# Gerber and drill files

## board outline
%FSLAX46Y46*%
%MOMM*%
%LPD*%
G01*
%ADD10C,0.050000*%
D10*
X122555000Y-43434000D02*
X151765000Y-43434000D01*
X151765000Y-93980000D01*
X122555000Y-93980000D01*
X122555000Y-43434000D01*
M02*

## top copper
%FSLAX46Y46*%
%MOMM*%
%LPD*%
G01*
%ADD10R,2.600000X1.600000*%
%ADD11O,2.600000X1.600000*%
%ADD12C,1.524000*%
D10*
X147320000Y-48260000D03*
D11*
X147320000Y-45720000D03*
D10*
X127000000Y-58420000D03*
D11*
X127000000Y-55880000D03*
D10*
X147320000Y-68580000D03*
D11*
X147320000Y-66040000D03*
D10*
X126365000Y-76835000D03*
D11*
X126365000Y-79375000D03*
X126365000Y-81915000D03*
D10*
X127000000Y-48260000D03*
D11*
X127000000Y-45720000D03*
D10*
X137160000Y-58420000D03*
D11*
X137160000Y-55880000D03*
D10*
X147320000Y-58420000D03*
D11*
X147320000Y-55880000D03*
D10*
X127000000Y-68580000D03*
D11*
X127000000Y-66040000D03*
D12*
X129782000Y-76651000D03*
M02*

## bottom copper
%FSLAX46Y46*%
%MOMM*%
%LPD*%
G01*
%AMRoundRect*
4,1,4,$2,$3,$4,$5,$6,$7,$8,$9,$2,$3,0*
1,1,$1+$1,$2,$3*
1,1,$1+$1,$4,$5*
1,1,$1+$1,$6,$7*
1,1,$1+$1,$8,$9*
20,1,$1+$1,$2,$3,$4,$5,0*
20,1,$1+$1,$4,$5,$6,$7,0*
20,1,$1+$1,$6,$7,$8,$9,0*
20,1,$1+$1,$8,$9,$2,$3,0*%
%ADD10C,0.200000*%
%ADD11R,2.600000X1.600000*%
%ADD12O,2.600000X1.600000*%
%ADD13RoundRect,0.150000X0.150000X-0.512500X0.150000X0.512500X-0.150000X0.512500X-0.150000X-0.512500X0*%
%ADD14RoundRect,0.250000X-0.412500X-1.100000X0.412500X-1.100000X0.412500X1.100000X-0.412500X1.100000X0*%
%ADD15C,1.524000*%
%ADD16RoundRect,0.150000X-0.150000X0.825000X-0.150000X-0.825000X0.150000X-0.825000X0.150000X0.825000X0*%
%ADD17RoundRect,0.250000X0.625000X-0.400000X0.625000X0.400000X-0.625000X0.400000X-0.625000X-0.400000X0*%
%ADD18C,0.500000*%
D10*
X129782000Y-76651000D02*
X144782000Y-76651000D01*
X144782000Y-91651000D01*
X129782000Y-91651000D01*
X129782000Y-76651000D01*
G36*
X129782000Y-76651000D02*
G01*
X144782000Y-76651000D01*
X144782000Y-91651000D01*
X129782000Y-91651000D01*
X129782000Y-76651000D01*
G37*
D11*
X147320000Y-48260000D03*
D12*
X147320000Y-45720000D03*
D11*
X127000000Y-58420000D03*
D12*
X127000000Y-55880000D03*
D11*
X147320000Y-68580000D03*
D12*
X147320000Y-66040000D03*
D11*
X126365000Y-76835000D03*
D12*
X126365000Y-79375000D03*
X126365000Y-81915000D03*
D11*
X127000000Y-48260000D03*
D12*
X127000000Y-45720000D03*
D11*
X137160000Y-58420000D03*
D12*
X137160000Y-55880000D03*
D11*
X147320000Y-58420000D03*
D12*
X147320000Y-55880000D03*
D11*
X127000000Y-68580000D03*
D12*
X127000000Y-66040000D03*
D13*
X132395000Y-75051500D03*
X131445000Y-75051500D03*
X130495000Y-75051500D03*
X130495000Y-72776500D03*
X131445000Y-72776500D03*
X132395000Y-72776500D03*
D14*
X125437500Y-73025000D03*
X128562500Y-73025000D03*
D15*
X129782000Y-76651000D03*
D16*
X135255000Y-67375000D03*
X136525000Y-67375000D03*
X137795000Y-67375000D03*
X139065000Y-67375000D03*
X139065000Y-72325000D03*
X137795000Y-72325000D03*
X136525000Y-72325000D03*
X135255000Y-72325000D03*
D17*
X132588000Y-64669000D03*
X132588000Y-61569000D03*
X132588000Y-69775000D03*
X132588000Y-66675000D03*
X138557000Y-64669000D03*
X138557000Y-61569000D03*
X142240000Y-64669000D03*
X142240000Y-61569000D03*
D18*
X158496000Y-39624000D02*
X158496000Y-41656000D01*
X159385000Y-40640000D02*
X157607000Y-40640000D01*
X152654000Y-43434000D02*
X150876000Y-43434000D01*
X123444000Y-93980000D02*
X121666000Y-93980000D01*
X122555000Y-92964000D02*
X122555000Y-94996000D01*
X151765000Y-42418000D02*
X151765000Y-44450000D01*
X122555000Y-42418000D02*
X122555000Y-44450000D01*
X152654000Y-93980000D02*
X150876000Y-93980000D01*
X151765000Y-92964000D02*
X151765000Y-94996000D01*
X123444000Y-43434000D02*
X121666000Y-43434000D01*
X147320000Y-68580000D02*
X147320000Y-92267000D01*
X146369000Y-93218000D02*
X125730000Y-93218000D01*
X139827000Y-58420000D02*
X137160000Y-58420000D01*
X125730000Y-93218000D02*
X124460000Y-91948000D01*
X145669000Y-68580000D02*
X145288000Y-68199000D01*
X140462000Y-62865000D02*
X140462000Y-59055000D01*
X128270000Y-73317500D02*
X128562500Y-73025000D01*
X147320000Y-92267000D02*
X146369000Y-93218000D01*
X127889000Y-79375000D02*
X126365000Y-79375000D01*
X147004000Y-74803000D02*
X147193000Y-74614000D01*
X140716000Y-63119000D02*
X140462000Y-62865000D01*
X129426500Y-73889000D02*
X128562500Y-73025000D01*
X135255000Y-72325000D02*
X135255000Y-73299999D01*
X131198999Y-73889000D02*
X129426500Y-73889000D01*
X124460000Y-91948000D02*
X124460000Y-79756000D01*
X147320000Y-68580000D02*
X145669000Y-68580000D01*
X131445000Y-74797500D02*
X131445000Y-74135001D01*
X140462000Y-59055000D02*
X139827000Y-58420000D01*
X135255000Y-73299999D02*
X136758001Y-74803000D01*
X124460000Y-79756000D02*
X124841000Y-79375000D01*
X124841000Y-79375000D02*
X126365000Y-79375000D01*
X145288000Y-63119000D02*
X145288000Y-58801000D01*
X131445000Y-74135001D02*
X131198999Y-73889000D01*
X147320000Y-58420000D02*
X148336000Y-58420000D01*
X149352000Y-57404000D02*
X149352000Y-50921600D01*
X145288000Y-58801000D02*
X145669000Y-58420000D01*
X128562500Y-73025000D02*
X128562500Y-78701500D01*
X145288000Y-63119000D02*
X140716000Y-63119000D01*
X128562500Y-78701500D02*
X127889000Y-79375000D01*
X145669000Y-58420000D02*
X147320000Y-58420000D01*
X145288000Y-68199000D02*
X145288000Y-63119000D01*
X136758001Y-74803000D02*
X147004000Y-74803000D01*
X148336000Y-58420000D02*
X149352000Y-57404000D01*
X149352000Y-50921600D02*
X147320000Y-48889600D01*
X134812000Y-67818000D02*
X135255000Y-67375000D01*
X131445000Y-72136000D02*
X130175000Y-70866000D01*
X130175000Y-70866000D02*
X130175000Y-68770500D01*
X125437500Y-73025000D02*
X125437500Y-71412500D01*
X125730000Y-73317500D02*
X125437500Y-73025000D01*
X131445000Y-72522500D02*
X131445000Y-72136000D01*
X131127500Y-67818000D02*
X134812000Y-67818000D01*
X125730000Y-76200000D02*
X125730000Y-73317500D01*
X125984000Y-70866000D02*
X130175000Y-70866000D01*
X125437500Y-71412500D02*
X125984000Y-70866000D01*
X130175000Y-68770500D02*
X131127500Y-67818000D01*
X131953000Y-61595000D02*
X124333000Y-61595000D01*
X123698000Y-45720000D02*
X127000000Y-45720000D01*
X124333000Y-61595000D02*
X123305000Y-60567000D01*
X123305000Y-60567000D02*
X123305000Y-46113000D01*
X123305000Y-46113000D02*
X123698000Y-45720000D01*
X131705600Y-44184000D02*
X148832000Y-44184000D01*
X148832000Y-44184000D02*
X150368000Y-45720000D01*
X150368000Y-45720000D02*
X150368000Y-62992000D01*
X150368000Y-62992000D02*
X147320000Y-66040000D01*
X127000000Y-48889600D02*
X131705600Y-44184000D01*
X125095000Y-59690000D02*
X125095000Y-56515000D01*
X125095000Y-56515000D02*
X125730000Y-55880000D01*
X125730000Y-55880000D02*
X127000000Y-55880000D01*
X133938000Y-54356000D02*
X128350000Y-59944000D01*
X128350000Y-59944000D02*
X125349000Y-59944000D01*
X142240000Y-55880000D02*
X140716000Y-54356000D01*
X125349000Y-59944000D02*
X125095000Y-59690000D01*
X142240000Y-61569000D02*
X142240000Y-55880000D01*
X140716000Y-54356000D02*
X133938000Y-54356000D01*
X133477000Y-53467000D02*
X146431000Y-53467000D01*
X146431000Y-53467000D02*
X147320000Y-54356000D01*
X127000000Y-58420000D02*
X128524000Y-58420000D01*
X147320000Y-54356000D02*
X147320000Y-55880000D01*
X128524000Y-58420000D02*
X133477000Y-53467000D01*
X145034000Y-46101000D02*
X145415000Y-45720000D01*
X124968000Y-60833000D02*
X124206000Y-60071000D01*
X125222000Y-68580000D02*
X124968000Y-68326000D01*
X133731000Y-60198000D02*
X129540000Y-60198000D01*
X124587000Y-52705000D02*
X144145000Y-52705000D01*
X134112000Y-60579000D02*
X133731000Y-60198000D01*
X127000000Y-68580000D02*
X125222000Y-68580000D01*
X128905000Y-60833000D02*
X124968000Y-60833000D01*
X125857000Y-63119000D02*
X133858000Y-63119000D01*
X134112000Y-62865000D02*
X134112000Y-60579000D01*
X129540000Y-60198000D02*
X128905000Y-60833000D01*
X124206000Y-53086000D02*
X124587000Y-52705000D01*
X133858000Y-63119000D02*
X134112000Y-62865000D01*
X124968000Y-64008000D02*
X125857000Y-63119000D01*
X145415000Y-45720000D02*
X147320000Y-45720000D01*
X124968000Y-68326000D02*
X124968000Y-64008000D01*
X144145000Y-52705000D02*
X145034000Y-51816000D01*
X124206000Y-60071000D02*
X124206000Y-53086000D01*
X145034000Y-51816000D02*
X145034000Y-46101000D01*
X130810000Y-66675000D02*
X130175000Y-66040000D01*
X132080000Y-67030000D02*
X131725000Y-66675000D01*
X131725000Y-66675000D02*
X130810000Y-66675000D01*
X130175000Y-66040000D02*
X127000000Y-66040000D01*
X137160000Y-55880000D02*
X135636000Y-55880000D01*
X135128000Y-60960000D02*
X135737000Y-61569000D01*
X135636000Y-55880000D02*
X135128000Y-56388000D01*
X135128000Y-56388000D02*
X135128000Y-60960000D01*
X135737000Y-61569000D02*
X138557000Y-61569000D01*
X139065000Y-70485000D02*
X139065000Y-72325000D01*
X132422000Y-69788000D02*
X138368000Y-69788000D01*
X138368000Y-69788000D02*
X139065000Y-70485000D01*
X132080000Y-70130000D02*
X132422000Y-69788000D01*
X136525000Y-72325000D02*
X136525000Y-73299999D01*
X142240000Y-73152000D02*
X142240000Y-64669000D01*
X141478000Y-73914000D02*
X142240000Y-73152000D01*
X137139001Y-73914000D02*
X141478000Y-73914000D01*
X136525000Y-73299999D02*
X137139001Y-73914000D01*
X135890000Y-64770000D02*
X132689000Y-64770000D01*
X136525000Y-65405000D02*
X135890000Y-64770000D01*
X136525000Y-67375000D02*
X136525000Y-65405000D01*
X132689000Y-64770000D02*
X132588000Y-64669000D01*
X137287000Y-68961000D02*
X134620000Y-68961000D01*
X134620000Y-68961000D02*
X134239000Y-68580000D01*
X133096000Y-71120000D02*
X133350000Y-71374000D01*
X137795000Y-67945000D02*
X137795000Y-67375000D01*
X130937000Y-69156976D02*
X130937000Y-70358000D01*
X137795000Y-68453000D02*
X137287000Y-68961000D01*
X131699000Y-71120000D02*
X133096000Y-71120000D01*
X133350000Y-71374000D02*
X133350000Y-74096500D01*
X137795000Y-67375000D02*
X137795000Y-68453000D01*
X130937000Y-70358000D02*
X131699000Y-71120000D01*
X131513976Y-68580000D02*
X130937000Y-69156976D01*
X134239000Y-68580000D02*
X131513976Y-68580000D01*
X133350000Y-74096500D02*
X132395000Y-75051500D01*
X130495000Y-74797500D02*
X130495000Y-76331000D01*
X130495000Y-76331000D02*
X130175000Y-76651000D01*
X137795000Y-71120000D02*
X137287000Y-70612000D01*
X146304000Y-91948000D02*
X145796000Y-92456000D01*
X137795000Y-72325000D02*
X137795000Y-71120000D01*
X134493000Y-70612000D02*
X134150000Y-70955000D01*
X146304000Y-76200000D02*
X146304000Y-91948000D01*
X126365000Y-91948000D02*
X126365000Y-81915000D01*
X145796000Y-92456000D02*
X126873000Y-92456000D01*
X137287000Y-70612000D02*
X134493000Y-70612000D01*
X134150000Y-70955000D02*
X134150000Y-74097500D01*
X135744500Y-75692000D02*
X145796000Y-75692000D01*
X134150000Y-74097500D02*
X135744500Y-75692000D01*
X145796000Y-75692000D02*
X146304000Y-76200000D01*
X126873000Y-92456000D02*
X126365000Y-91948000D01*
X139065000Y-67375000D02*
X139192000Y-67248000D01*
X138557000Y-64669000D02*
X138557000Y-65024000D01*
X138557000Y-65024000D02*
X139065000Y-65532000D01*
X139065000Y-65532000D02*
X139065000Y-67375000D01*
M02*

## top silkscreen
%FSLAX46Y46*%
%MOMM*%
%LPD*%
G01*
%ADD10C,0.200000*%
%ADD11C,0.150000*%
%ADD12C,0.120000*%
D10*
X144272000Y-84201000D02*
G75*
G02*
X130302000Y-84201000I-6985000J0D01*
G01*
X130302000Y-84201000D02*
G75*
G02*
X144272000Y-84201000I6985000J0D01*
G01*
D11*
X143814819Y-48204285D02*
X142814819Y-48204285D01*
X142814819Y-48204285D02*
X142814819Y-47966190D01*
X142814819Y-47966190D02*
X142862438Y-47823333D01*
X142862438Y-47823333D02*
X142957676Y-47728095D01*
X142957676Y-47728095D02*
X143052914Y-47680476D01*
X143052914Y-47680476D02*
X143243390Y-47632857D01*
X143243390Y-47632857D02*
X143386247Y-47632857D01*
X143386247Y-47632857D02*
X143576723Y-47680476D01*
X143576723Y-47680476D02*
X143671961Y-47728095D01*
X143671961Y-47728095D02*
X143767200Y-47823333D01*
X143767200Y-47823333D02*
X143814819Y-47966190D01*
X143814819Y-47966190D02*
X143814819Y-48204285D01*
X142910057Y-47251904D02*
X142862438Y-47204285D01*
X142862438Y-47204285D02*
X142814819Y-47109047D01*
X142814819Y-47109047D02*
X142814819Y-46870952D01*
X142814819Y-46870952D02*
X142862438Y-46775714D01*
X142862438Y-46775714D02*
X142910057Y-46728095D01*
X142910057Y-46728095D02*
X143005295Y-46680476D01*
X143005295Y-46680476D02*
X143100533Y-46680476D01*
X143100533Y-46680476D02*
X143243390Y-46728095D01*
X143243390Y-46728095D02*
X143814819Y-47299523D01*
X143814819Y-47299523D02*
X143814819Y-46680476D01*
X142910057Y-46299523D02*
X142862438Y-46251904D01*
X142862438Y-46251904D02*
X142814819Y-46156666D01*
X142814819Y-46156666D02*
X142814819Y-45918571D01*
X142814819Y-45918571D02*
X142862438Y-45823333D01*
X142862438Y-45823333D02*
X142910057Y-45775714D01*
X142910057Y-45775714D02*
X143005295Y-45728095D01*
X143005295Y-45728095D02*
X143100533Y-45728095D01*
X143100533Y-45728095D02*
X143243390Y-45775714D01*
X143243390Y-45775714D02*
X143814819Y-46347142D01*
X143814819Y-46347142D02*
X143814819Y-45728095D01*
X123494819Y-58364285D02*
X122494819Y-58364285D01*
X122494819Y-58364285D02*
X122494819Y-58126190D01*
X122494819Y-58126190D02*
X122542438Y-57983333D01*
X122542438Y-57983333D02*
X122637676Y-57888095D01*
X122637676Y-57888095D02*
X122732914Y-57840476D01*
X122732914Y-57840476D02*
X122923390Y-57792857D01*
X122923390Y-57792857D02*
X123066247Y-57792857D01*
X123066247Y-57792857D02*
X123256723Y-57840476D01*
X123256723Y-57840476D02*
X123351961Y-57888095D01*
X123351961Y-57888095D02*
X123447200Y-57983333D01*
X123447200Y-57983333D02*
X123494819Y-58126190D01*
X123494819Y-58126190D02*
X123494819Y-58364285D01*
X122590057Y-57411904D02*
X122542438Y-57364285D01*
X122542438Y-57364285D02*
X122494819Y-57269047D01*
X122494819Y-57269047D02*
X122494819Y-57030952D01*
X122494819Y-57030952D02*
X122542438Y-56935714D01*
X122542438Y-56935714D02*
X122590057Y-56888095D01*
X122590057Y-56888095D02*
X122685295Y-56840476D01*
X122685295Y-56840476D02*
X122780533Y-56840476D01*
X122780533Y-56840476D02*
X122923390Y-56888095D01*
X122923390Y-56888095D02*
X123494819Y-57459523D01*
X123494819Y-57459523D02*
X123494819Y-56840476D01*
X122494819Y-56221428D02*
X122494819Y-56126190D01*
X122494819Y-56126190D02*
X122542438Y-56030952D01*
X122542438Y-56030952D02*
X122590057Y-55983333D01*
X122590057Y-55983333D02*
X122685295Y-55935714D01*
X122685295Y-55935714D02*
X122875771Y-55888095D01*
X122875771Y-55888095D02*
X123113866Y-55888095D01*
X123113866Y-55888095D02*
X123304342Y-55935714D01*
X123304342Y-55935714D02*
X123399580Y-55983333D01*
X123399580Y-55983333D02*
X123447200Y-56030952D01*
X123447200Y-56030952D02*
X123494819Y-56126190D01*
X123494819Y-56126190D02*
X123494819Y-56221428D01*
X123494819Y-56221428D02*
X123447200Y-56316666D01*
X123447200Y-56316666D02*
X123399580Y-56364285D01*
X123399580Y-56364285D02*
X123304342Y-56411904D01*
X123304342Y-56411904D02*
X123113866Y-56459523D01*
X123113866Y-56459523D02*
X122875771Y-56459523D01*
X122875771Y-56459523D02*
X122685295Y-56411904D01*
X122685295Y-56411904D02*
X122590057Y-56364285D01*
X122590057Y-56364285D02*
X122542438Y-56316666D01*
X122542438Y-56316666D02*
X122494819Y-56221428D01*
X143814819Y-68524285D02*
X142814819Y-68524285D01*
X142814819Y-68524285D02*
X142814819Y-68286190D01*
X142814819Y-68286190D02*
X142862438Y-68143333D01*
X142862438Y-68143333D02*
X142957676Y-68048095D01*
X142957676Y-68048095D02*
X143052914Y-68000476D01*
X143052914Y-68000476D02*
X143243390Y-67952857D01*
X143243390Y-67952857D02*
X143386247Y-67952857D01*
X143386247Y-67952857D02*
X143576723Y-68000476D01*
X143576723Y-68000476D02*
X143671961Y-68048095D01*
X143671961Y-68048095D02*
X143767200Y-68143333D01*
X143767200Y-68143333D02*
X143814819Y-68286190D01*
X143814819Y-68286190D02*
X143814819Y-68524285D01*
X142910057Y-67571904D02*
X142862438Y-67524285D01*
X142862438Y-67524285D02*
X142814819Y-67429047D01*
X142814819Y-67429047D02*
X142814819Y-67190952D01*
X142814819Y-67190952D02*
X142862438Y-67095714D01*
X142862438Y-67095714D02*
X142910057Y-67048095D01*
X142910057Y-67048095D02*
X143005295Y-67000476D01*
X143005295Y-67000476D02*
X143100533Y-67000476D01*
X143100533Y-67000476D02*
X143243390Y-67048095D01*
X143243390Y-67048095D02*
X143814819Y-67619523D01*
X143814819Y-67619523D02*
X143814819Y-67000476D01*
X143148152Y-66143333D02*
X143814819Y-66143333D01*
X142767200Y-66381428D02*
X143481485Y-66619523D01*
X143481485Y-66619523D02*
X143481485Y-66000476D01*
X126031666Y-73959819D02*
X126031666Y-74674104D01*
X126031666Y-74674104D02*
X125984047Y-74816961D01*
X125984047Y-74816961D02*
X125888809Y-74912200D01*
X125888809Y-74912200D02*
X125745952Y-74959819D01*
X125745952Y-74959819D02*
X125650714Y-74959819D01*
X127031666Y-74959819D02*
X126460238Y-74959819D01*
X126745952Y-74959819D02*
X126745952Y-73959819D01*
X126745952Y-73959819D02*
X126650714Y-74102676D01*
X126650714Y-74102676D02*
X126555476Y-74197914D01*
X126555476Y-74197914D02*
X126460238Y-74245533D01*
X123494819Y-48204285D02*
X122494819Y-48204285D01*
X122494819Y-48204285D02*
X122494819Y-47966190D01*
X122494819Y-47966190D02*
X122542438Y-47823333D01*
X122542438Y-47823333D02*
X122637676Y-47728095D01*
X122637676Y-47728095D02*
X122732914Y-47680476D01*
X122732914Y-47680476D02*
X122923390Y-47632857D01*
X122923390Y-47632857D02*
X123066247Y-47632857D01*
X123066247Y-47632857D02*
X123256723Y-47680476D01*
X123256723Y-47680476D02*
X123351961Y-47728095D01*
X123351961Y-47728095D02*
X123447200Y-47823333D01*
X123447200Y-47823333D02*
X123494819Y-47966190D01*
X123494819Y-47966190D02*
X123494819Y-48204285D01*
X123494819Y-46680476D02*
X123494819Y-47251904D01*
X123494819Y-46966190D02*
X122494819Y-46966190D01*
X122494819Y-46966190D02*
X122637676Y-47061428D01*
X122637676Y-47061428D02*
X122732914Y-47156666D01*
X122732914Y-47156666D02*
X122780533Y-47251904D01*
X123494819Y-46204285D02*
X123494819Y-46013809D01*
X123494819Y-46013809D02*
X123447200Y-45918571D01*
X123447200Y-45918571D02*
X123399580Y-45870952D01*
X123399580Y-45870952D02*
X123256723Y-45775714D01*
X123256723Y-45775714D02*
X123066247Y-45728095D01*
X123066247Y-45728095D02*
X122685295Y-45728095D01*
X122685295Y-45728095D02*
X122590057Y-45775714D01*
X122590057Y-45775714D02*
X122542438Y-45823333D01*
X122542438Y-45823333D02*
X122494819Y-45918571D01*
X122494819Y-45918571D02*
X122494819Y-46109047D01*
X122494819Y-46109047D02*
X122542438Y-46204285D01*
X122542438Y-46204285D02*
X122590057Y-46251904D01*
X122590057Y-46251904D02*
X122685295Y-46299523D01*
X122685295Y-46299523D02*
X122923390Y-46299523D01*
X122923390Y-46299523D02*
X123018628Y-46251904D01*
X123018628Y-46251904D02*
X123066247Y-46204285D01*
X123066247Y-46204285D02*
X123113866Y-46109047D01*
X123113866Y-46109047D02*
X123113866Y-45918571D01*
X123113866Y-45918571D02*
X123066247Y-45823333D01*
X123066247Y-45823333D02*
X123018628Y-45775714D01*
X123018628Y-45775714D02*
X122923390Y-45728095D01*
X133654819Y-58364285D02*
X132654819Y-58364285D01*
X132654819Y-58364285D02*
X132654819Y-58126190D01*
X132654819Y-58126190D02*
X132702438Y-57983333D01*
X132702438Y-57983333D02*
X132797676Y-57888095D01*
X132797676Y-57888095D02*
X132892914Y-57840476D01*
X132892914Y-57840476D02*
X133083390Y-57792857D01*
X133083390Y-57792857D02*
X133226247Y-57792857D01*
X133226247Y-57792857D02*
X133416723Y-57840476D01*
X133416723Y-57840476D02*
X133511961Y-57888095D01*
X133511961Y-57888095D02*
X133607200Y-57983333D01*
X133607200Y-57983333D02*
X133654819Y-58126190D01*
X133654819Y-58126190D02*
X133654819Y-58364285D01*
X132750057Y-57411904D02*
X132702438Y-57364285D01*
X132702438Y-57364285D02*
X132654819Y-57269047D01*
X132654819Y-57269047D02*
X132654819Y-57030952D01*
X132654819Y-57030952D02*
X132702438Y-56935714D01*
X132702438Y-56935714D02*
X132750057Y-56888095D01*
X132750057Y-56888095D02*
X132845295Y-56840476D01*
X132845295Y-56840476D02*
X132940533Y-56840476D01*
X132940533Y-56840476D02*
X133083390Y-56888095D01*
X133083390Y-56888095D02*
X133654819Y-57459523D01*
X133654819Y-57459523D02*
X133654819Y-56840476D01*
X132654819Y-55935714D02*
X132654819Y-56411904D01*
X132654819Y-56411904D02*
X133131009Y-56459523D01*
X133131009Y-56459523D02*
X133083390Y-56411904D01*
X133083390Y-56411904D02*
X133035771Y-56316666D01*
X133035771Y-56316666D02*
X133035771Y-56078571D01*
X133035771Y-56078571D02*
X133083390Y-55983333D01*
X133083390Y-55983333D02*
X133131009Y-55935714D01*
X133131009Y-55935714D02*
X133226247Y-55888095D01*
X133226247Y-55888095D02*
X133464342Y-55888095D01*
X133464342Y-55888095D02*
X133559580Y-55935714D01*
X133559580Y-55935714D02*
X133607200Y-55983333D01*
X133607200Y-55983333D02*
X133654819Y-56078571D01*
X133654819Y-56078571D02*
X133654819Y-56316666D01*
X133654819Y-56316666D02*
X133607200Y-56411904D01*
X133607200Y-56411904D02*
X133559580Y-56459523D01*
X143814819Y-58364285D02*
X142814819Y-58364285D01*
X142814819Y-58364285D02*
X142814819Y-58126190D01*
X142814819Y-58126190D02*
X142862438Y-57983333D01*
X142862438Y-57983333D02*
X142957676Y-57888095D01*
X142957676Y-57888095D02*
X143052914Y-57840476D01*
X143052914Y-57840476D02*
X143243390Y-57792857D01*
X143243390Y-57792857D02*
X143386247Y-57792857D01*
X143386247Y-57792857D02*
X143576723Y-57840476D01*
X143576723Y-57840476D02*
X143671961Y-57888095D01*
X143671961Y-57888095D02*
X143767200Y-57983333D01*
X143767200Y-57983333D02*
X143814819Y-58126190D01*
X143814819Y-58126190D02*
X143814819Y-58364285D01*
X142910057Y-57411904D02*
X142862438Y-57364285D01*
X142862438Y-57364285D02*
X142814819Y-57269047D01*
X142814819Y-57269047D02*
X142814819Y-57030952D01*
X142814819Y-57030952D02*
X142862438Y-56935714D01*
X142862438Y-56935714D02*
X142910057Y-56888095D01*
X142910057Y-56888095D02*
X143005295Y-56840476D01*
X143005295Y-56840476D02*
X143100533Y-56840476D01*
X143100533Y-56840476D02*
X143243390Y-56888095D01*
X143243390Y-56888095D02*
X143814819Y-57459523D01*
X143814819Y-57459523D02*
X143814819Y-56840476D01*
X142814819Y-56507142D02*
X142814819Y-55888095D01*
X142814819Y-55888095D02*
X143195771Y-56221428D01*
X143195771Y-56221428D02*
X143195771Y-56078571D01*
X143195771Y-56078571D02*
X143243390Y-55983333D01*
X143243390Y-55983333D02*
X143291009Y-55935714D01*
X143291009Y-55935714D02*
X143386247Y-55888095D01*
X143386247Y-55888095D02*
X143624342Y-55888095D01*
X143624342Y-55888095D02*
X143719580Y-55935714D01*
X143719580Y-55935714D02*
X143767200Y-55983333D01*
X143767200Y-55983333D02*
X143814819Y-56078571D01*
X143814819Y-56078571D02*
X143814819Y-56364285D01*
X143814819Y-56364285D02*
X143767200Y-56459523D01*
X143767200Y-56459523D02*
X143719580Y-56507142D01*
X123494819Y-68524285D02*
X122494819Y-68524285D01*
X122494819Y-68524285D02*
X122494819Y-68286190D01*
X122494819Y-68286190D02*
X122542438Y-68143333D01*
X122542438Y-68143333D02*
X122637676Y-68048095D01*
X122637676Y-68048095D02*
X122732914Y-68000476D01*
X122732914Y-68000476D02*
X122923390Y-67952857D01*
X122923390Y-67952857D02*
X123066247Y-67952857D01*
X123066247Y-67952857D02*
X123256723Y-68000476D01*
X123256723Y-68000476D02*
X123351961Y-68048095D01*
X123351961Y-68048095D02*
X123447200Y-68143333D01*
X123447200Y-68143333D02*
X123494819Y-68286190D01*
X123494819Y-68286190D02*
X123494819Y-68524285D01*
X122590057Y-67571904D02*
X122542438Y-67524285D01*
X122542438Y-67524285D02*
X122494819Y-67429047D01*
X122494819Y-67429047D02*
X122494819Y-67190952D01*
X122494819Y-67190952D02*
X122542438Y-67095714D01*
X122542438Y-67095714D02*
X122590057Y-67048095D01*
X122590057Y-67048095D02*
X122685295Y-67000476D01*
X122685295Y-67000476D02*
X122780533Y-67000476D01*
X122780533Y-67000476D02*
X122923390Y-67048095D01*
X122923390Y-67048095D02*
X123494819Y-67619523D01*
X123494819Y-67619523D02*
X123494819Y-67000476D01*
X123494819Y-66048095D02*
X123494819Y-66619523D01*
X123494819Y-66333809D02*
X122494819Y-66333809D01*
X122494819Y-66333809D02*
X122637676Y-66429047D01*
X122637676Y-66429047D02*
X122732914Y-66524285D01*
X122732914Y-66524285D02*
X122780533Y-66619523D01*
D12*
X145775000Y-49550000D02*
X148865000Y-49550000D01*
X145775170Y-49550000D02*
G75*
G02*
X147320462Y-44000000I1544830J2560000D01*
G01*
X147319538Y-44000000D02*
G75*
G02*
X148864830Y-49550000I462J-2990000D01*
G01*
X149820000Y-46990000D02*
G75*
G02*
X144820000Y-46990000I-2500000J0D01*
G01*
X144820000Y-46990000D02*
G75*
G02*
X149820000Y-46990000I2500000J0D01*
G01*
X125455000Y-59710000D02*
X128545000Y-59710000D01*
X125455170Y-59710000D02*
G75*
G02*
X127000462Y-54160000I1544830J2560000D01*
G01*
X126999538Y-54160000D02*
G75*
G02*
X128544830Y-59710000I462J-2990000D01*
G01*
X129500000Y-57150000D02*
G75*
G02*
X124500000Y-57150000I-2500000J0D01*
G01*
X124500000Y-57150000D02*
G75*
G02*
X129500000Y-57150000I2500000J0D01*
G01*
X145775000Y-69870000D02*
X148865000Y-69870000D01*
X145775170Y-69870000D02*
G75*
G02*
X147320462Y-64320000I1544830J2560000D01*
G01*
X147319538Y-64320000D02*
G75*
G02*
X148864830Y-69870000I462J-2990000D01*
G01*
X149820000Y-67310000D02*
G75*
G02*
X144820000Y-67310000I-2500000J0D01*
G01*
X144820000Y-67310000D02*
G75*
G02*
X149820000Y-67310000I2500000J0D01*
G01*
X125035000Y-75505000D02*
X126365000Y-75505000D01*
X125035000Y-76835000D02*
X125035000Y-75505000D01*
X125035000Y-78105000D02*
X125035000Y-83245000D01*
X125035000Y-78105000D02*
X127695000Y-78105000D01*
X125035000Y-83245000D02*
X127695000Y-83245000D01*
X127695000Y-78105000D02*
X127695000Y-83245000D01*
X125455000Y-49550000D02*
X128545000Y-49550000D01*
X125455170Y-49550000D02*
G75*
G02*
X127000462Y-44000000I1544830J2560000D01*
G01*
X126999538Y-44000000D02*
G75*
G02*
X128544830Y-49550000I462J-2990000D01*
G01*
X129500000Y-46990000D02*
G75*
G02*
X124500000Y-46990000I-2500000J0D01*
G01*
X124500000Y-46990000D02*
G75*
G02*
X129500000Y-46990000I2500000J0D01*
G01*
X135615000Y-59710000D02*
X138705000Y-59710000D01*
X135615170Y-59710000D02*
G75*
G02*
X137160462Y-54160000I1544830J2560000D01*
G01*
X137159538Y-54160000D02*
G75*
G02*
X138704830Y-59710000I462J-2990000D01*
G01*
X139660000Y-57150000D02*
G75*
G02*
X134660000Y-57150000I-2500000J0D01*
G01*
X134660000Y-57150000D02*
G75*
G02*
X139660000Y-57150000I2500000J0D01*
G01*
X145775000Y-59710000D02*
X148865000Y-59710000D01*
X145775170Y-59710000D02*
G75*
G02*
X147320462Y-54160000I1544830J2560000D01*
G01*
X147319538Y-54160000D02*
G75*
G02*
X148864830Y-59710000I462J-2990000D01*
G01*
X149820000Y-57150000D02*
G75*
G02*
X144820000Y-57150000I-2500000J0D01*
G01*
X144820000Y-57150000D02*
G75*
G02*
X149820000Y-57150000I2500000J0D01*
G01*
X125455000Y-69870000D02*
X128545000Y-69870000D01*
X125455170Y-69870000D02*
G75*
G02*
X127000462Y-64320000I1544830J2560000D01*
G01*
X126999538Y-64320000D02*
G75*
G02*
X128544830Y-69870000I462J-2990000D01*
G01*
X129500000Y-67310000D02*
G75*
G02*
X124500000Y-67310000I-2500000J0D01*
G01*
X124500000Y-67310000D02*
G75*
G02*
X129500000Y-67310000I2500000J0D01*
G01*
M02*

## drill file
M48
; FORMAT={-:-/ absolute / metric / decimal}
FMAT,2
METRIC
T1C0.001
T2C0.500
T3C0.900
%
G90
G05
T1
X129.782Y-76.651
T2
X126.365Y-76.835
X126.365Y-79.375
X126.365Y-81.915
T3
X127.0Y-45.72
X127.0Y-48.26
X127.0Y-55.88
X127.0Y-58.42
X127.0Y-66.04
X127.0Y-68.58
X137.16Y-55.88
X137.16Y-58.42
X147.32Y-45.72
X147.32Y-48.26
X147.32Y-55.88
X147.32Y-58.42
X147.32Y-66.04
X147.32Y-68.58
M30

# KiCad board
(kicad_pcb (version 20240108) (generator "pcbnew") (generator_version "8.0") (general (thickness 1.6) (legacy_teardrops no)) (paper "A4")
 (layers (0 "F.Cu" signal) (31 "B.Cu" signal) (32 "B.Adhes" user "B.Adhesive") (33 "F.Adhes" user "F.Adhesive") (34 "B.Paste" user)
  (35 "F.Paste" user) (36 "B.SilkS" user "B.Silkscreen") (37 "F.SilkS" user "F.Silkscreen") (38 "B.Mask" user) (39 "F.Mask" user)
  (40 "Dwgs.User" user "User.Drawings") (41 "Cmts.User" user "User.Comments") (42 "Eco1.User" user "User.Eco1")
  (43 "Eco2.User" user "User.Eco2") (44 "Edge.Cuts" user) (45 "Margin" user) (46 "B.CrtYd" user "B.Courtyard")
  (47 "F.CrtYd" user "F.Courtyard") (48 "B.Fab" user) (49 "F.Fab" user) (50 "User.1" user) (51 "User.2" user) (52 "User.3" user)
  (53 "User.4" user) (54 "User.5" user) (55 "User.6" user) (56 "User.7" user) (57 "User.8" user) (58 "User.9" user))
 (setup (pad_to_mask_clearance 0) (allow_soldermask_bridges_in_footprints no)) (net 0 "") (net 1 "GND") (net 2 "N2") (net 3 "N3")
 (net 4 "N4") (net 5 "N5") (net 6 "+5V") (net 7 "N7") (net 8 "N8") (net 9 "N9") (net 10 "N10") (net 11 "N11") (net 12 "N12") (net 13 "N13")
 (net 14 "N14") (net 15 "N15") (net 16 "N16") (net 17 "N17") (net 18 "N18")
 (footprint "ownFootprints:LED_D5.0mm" (layer "F.Cu") (at 147.32 48.26 90)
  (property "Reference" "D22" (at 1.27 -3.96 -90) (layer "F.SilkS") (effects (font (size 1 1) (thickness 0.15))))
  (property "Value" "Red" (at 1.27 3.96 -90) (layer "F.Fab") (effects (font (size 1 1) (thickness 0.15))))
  (fp_line (start -1.29 -1.545) (end -1.29 1.545) (stroke (width 0.12) (type solid)) (layer "F.SilkS"))
  (fp_arc (start -1.29 -1.54483) (mid 2.072002 -2.880433) (end 4.26 0.000462) (stroke (width 0.12) (type solid)) (layer "F.SilkS"))
  (fp_arc (start 4.26 -0.000462) (mid 2.072002 2.880433) (end -1.29 1.54483) (stroke (width 0.12) (type solid)) (layer "F.SilkS"))
  (fp_circle (center 1.27 0) (end 3.77 0) (stroke (width 0.12) (type solid)) (fill none) (layer "F.SilkS"))
  (pad "1" thru_hole rect (at 0 0 90) (size 1.6 2.6) (drill 0.9) (layers "*.Cu" "*.Mask") (remove_unused_layers no) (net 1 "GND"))
  (pad "2" thru_hole oval (at 2.54 0 90) (size 1.6 2.6) (drill 0.9) (layers "*.Cu" "*.Mask") (remove_unused_layers no) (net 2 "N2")))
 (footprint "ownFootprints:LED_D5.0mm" (layer "F.Cu") (at 127 58.42 90)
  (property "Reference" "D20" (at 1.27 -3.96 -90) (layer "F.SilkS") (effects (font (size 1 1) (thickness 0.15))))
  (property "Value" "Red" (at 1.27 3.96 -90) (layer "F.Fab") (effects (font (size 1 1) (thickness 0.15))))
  (fp_line (start -1.29 -1.545) (end -1.29 1.545) (stroke (width 0.12) (type solid)) (layer "F.SilkS"))
  (fp_arc (start -1.29 -1.54483) (mid 2.072002 -2.880433) (end 4.26 0.000462) (stroke (width 0.12) (type solid)) (layer "F.SilkS"))
  (fp_arc (start 4.26 -0.000462) (mid 2.072002 2.880433) (end -1.29 1.54483) (stroke (width 0.12) (type solid)) (layer "F.SilkS"))
  (fp_circle (center 1.27 0) (end 3.77 0) (stroke (width 0.12) (type solid)) (fill none) (layer "F.SilkS"))
  (pad "1" thru_hole rect (at 0 0 90) (size 1.6 2.6) (drill 0.9) (layers "*.Cu" "*.Mask") (remove_unused_layers no) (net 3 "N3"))
  (pad "2" thru_hole oval (at 2.54 0 90) (size 1.6 2.6) (drill 0.9) (layers "*.Cu" "*.Mask") (remove_unused_layers no) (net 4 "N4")))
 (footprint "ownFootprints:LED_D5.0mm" (layer "F.Cu") (at 147.32 68.58 90)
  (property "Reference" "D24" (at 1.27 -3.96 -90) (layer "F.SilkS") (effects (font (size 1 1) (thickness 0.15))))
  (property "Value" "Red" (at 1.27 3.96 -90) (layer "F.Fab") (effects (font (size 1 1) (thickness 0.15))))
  (fp_line (start -1.29 -1.545) (end -1.29 1.545) (stroke (width 0.12) (type solid)) (layer "F.SilkS"))
  (fp_arc (start -1.29 -1.54483) (mid 2.072002 -2.880433) (end 4.26 0.000462) (stroke (width 0.12) (type solid)) (layer "F.SilkS"))
  (fp_arc (start 4.26 -0.000462) (mid 2.072002 2.880433) (end -1.29 1.54483) (stroke (width 0.12) (type solid)) (layer "F.SilkS"))
  (fp_circle (center 1.27 0) (end 3.77 0) (stroke (width 0.12) (type solid)) (fill none) (layer "F.SilkS"))
  (pad "1" thru_hole rect (at 0 0 90) (size 1.6 2.6) (drill 0.9) (layers "*.Cu" "*.Mask") (remove_unused_layers no) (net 1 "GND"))
  (pad "2" thru_hole oval (at 2.54 0 90) (size 1.6 2.6) (drill 0.9) (layers "*.Cu" "*.Mask") (remove_unused_layers no) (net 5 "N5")))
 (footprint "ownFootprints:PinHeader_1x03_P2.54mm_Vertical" (layer "F.Cu") (at 126.365 76.835)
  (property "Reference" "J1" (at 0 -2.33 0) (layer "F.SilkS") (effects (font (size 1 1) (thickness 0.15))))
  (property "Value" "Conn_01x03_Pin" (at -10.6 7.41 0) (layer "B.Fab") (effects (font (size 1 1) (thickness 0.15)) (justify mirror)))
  (fp_line (start -1.33 -1.33) (end 0 -1.33) (stroke (width 0.12) (type solid)) (layer "F.SilkS"))
  (fp_line (start -1.33 0) (end -1.33 -1.33) (stroke (width 0.12) (type solid)) (layer "F.SilkS"))
  (fp_line (start -1.33 1.27) (end -1.33 6.41) (stroke (width 0.12) (type solid)) (layer "F.SilkS"))
  (fp_line (start -1.33 1.27) (end 1.33 1.27) (stroke (width 0.12) (type solid)) (layer "F.SilkS"))
  (fp_line (start -1.33 6.41) (end 1.33 6.41) (stroke (width 0.12) (type solid)) (layer "F.SilkS"))
  (fp_line (start 1.33 1.27) (end 1.33 6.41) (stroke (width 0.12) (type solid)) (layer "F.SilkS"))
  (pad "1" thru_hole rect (at 0 0) (size 2.6 1.6) (drill 0.5) (layers "*.Cu" "*.Mask") (remove_unused_layers no) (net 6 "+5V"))
  (pad "2" thru_hole oval (at 0 2.54) (size 2.6 1.6) (drill 0.5) (layers "*.Cu" "*.Mask") (remove_unused_layers no) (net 1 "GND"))
  (pad "3" thru_hole oval (at 0 5.08) (size 2.6 1.6) (drill 0.5) (layers "*.Cu" "*.Mask") (remove_unused_layers no) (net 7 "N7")))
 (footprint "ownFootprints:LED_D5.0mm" (layer "F.Cu") (at 127 48.26 90)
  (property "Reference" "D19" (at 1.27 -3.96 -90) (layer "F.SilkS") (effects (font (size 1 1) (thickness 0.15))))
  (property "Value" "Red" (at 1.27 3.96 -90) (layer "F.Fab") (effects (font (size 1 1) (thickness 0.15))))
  (fp_line (start -1.29 -1.545) (end -1.29 1.545) (stroke (width 0.12) (type solid)) (layer "F.SilkS"))
  (fp_arc (start -1.29 -1.54483) (mid 2.072002 -2.880433) (end 4.26 0.000462) (stroke (width 0.12) (type solid)) (layer "F.SilkS"))
  (fp_arc (start 4.26 -0.000462) (mid 2.072002 2.880433) (end -1.29 1.54483) (stroke (width 0.12) (type solid)) (layer "F.SilkS"))
  (fp_circle (center 1.27 0) (end 3.77 0) (stroke (width 0.12) (type solid)) (fill none) (layer "F.SilkS"))
  (pad "1" thru_hole rect (at 0 0 90) (size 1.6 2.6) (drill 0.9) (layers "*.Cu" "*.Mask") (remove_unused_layers no) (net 5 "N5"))
  (pad "2" thru_hole oval (at 2.54 0 90) (size 1.6 2.6) (drill 0.9) (layers "*.Cu" "*.Mask") (remove_unused_layers no) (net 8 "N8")))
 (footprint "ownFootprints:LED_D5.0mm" (layer "F.Cu") (at 137.16 58.42 90)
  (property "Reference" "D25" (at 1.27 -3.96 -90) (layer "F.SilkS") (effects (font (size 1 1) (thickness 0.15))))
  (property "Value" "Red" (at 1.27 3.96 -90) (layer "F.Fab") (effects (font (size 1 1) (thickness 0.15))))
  (fp_line (start -1.29 -1.545) (end -1.29 1.545) (stroke (width 0.12) (type solid)) (layer "F.SilkS"))
  (fp_arc (start -1.29 -1.54483) (mid 2.072002 -2.880433) (end 4.26 0.000462) (stroke (width 0.12) (type solid)) (layer "F.SilkS"))
  (fp_arc (start 4.26 -0.000462) (mid 2.072002 2.880433) (end -1.29 1.54483) (stroke (width 0.12) (type solid)) (layer "F.SilkS"))
  (fp_circle (center 1.27 0) (end 3.77 0) (stroke (width 0.12) (type solid)) (fill none) (layer "F.SilkS"))
  (pad "1" thru_hole rect (at 0 0 90) (size 1.6 2.6) (drill 0.9) (layers "*.Cu" "*.Mask") (remove_unused_layers no) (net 1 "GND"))
  (pad "2" thru_hole oval (at 2.54 0 90) (size 1.6 2.6) (drill 0.9) (layers "*.Cu" "*.Mask") (remove_unused_layers no) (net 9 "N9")))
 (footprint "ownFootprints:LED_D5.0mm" (layer "F.Cu") (at 147.32 58.42 90)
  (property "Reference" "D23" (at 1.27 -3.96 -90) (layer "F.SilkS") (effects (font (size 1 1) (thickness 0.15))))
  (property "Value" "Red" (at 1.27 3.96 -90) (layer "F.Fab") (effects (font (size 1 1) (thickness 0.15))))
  (fp_line (start -1.29 -1.545) (end -1.29 1.545) (stroke (width 0.12) (type solid)) (layer "F.SilkS"))
  (fp_arc (start -1.29 -1.54483) (mid 2.072002 -2.880433) (end 4.26 0.000462) (stroke (width 0.12) (type solid)) (layer "F.SilkS"))
  (fp_arc (start 4.26 -0.000462) (mid 2.072002 2.880433) (end -1.29 1.54483) (stroke (width 0.12) (type solid)) (layer "F.SilkS"))
  (fp_circle (center 1.27 0) (end 3.77 0) (stroke (width 0.12) (type solid)) (fill none) (layer "F.SilkS"))
  (pad "1" thru_hole rect (at 0 0 90) (size 1.6 2.6) (drill 0.9) (layers "*.Cu" "*.Mask") (remove_unused_layers no) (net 1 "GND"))
  (pad "2" thru_hole oval (at 2.54 0 90) (size 1.6 2.6) (drill 0.9) (layers "*.Cu" "*.Mask") (remove_unused_layers no) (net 3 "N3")))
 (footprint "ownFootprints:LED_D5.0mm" (layer "F.Cu") (at 127 68.58 90)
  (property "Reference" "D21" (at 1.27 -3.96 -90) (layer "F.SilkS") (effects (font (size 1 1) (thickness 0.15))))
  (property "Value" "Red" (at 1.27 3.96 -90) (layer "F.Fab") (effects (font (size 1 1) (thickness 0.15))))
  (fp_line (start -1.29 -1.545) (end -1.29 1.545) (stroke (width 0.12) (type solid)) (layer "F.SilkS"))
  (fp_arc (start -1.29 -1.54483) (mid 2.072002 -2.880433) (end 4.26 0.000462) (stroke (width 0.12) (type solid)) (layer "F.SilkS"))
  (fp_arc (start 4.26 -0.000462) (mid 2.072002 2.880433) (end -1.29 1.54483) (stroke (width 0.12) (type solid)) (layer "F.SilkS"))
  (fp_circle (center 1.27 0) (end 3.77 0) (stroke (width 0.12) (type solid)) (fill none) (layer "F.SilkS"))
  (pad "1" thru_hole rect (at 0 0 90) (size 1.6 2.6) (drill 0.9) (layers "*.Cu" "*.Mask") (remove_unused_layers no) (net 2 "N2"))
  (pad "2" thru_hole oval (at 2.54 0 90) (size 1.6 2.6) (drill 0.9) (layers "*.Cu" "*.Mask") (remove_unused_layers no) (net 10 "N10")))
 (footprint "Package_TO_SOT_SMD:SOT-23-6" (layer "B.Cu") (at 131.445 73.914 90)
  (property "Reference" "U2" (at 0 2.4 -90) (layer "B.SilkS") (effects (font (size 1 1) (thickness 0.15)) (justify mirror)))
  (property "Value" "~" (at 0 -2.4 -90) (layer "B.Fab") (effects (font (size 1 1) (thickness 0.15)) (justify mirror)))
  (pad "1" smd roundrect (at -1.1375 0.95 90) (size 1.325 0.6) (layers "B.Cu" "B.Paste" "B.Mask") (roundrect_rratio 0.25) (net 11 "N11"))
  (pad "2" smd roundrect (at -1.1375 0 90) (size 1.325 0.6) (layers "B.Cu" "B.Paste" "B.Mask") (roundrect_rratio 0.25) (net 1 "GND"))
  (pad "3" smd roundrect (at -1.1375 -0.95 90) (size 1.325 0.6) (layers "B.Cu" "B.Paste" "B.Mask") (roundrect_rratio 0.25) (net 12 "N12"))
  (pad "4" smd roundrect (at 1.1375 -0.95 90) (size 1.325 0.6) (layers "B.Cu" "B.Paste" "B.Mask") (roundrect_rratio 0.25) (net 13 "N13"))
  (pad "5" smd roundrect (at 1.1375 0 90) (size 1.325 0.6) (layers "B.Cu" "B.Paste" "B.Mask") (roundrect_rratio 0.25) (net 6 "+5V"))
  (pad "6" smd roundrect (at 1.1375 0.95 90) (size 1.325 0.6) (layers "B.Cu" "B.Paste" "B.Mask") (roundrect_rratio 0.25) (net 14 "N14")))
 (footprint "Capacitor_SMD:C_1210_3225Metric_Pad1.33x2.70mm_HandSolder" (layer "B.Cu") (at 127 73.025)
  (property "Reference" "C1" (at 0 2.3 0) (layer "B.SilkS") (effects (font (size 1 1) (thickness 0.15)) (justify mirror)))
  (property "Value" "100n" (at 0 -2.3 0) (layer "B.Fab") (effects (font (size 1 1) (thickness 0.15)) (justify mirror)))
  (pad "1" smd roundrect (at -1.5625 0) (size 1.325 2.7) (layers "B.Cu" "B.Paste" "B.Mask") (roundrect_rratio 0.188679) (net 6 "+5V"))
  (pad "2" smd roundrect (at 1.5625 0) (size 1.325 2.7) (layers "B.Cu" "B.Paste" "B.Mask") (roundrect_rratio 0.188679) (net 1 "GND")))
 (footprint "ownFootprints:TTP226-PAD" (layer "B.Cu") (at 119.782 80.651 -90)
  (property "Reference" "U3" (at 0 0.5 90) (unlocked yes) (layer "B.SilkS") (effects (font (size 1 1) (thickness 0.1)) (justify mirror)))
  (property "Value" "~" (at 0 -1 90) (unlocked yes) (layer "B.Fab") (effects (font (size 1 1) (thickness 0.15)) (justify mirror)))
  (fp_rect (start 11 -25) (end -4 -10) (stroke (width 0.2) (type solid)) (fill solid) (layer "B.Cu"))
  (pad "1" thru_hole circle (at -4 -10 270) (size 1.524 1.524) (drill 0.001) (layers "*.Cu" "B.Mask") (remove_unused_layers no)
   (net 12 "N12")))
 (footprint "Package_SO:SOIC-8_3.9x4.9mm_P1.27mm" (layer "B.Cu") (at 137.16 69.85 -90)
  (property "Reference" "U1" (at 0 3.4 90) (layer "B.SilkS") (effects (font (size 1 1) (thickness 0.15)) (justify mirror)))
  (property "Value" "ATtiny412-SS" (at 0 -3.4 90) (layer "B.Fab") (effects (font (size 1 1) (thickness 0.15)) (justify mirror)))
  (pad "1" smd roundrect (at -2.475 1.905 270) (size 1.95 0.6) (layers "B.Cu" "B.Paste" "B.Mask") (roundrect_rratio 0.25) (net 6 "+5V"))
  (pad "2" smd roundrect (at -2.475 0.635 270) (size 1.95 0.6) (layers "B.Cu" "B.Paste" "B.Mask") (roundrect_rratio 0.25) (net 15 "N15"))
  (pad "3" smd roundrect (at -2.475 -0.635 270) (size 1.95 0.6) (layers "B.Cu" "B.Paste" "B.Mask") (roundrect_rratio 0.25) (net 11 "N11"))
  (pad "4" smd roundrect (at -2.475 -1.905 270) (size 1.95 0.6) (layers "B.Cu" "B.Paste" "B.Mask") (roundrect_rratio 0.25) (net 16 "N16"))
  (pad "5" smd roundrect (at 2.475 -1.905 270) (size 1.95 0.6) (layers "B.Cu" "B.Paste" "B.Mask") (roundrect_rratio 0.25) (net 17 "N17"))
  (pad "6" smd roundrect (at 2.475 -0.635 270) (size 1.95 0.6) (layers "B.Cu" "B.Paste" "B.Mask") (roundrect_rratio 0.25) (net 7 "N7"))
  (pad "7" smd roundrect (at 2.475 0.635 270) (size 1.95 0.6) (layers "B.Cu" "B.Paste" "B.Mask") (roundrect_rratio 0.25) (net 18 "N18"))
  (pad "8" smd roundrect (at 2.475 1.905 270) (size 1.95 0.6) (layers "B.Cu" "B.Paste" "B.Mask") (roundrect_rratio 0.25) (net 1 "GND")))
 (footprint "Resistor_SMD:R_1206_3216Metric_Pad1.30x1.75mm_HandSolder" (layer "B.Cu") (at 132.588 63.119 90)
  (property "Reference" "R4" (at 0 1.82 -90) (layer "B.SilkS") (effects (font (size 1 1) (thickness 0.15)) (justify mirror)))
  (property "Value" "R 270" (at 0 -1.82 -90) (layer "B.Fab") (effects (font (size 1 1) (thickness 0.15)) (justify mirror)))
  (pad "1" smd roundrect (at -1.55 0 90) (size 1.3 1.75) (layers "B.Cu" "B.Paste" "B.Mask") (roundrect_rratio 0.192308) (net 15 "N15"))
  (pad "2" smd roundrect (at 1.55 0 90) (size 1.3 1.75) (layers "B.Cu" "B.Paste" "B.Mask") (roundrect_rratio 0.192308) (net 8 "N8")))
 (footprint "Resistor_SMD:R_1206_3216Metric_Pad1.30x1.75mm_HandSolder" (layer "B.Cu") (at 132.588 68.225 90)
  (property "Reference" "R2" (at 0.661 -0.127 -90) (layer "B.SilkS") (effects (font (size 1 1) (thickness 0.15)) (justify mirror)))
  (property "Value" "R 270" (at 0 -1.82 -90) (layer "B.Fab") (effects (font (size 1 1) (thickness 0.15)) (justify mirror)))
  (pad "1" smd roundrect (at -1.55 0 90) (size 1.3 1.75) (layers "B.Cu" "B.Paste" "B.Mask") (roundrect_rratio 0.192308) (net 17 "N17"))
  (pad "2" smd roundrect (at 1.55 0 90) (size 1.3 1.75) (layers "B.Cu" "B.Paste" "B.Mask") (roundrect_rratio 0.192308) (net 10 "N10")))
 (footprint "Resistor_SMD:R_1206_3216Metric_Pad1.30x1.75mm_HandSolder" (layer "B.Cu") (at 138.557 63.119 90)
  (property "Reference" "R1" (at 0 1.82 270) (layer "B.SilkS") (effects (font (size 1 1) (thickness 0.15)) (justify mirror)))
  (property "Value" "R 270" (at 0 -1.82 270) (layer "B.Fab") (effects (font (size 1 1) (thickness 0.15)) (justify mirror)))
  (pad "1" smd roundrect (at -1.55 0 90) (size 1.3 1.75) (layers "B.Cu" "B.Paste" "B.Mask") (roundrect_rratio 0.192308) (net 16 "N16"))
  (pad "2" smd roundrect (at 1.55 0 90) (size 1.3 1.75) (layers "B.Cu" "B.Paste" "B.Mask") (roundrect_rratio 0.192308) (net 9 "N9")))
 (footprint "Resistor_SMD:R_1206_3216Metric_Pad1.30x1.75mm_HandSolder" (layer "B.Cu") (at 142.24 63.119 90)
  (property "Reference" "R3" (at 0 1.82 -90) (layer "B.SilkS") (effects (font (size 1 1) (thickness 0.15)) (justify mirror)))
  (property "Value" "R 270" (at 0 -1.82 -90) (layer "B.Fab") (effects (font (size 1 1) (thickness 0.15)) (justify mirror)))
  (pad "1" smd roundrect (at -1.55 0 90) (size 1.3 1.75) (layers "B.Cu" "B.Paste" "B.Mask") (roundrect_rratio 0.192308) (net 18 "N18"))
  (pad "2" smd roundrect (at 1.55 0 90) (size 1.3 1.75) (layers "B.Cu" "B.Paste" "B.Mask") (roundrect_rratio 0.192308) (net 4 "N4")))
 (gr_circle (center 137.287 84.201) (end 144.272 84.201) (stroke (width 0.2) (type default)) (fill none) (layer "F.SilkS"))
 (gr_rect (start 122.555 43.434) (end 151.765 93.98) (stroke (width 0.05) (type default)) (fill none) (layer "Edge.Cuts"))
 (segment (start 158.496 39.624) (end 158.496 41.656) (width 0.5) (layer "B.Cu") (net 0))
 (segment (start 159.385 40.64) (end 157.607 40.64) (width 0.5) (layer "B.Cu") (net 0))
 (segment (start 152.654 43.434) (end 150.876 43.434) (width 0.5) (layer "B.Cu") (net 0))
 (segment (start 123.444 93.98) (end 121.666 93.98) (width 0.5) (layer "B.Cu") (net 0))
 (segment (start 122.555 92.964) (end 122.555 94.996) (width 0.5) (layer "B.Cu") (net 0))
 (segment (start 151.765 42.418) (end 151.765 44.45) (width 0.5) (layer "B.Cu") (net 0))
 (segment (start 122.555 42.418) (end 122.555 44.45) (width 0.5) (layer "B.Cu") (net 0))
 (segment (start 152.654 93.98) (end 150.876 93.98) (width 0.5) (layer "B.Cu") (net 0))
 (segment (start 151.765 92.964) (end 151.765 94.996) (width 0.5) (layer "B.Cu") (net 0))
 (segment (start 123.444 43.434) (end 121.666 43.434) (width 0.5) (layer "B.Cu") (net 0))
 (segment (start 147.32 68.58) (end 147.32 92.267) (width 0.5) (layer "B.Cu") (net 1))
 (segment (start 146.369 93.218) (end 125.73 93.218) (width 0.5) (layer "B.Cu") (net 1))
 (segment (start 139.827 58.42) (end 137.16 58.42) (width 0.5) (layer "B.Cu") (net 1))
 (segment (start 125.73 93.218) (end 124.46 91.948) (width 0.5) (layer "B.Cu") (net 1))
 (segment (start 145.669 68.58) (end 145.288 68.199) (width 0.5) (layer "B.Cu") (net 1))
 (segment (start 140.462 62.865) (end 140.462 59.055) (width 0.5) (layer "B.Cu") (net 1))
 (segment (start 128.27 73.3175) (end 128.5625 73.025) (width 0.5) (layer "B.Cu") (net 1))
 (segment (start 147.32 92.267) (end 146.369 93.218) (width 0.5) (layer "B.Cu") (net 1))
 (segment (start 127.889 79.375) (end 126.365 79.375) (width 0.5) (layer "B.Cu") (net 1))
 (segment (start 147.004 74.803) (end 147.193 74.614) (width 0.5) (layer "B.Cu") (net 1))
 (segment (start 140.716 63.119) (end 140.462 62.865) (width 0.5) (layer "B.Cu") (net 1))
 (segment (start 129.4265 73.889) (end 128.5625 73.025) (width 0.5) (layer "B.Cu") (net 1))
 (segment (start 135.255 72.325) (end 135.255 73.299999) (width 0.5) (layer "B.Cu") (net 1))
 (segment (start 131.198999 73.889) (end 129.4265 73.889) (width 0.5) (layer "B.Cu") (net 1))
 (segment (start 124.46 91.948) (end 124.46 79.756) (width 0.5) (layer "B.Cu") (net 1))
 (segment (start 147.32 68.58) (end 145.669 68.58) (width 0.5) (layer "B.Cu") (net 1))
 (segment (start 131.445 74.7975) (end 131.445 74.135001) (width 0.5) (layer "B.Cu") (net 1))
 (segment (start 140.462 59.055) (end 139.827 58.42) (width 0.5) (layer "B.Cu") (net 1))
 (segment (start 135.255 73.299999) (end 136.758001 74.803) (width 0.5) (layer "B.Cu") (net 1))
 (segment (start 124.46 79.756) (end 124.841 79.375) (width 0.5) (layer "B.Cu") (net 1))
 (segment (start 124.841 79.375) (end 126.365 79.375) (width 0.5) (layer "B.Cu") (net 1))
 (segment (start 145.288 63.119) (end 145.288 58.801) (width 0.5) (layer "B.Cu") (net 1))
 (segment (start 131.445 74.135001) (end 131.198999 73.889) (width 0.5) (layer "B.Cu") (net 1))
 (segment (start 147.32 58.42) (end 148.336 58.42) (width 0.5) (layer "B.Cu") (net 1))
 (segment (start 149.352 57.404) (end 149.352 50.9216) (width 0.5) (layer "B.Cu") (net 1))
 (segment (start 145.288 58.801) (end 145.669 58.42) (width 0.5) (layer "B.Cu") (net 1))
 (segment (start 128.5625 73.025) (end 128.5625 78.7015) (width 0.5) (layer "B.Cu") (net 1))
 (segment (start 145.288 63.119) (end 140.716 63.119) (width 0.5) (layer "B.Cu") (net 1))
 (segment (start 128.5625 78.7015) (end 127.889 79.375) (width 0.5) (layer "B.Cu") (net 1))
 (segment (start 145.669 58.42) (end 147.32 58.42) (width 0.5) (layer "B.Cu") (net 1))
 (segment (start 145.288 68.199) (end 145.288 63.119) (width 0.5) (layer "B.Cu") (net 1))
 (segment (start 136.758001 74.803) (end 147.004 74.803) (width 0.5) (layer "B.Cu") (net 1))
 (segment (start 148.336 58.42) (end 149.352 57.404) (width 0.5) (layer "B.Cu") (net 1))
 (segment (start 149.352 50.9216) (end 147.32 48.8896) (width 0.5) (layer "B.Cu") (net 1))
 (segment (start 134.812 67.818) (end 135.255 67.375) (width 0.5) (layer "B.Cu") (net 6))
 (segment (start 131.445 72.136) (end 130.175 70.866) (width 0.5) (layer "B.Cu") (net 6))
 (segment (start 130.175 70.866) (end 130.175 68.7705) (width 0.5) (layer "B.Cu") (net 6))
 (segment (start 125.4375 73.025) (end 125.4375 71.4125) (width 0.5) (layer "B.Cu") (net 6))
 (segment (start 125.73 73.3175) (end 125.4375 73.025) (width 0.5) (layer "B.Cu") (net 6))
 (segment (start 131.445 72.5225) (end 131.445 72.136) (width 0.5) (layer "B.Cu") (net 6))
 (segment (start 131.1275 67.818) (end 134.812 67.818) (width 0.5) (layer "B.Cu") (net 6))
 (segment (start 125.73 76.2) (end 125.73 73.3175) (width 0.5) (layer "B.Cu") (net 6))
 (segment (start 125.984 70.866) (end 130.175 70.866) (width 0.5) (layer "B.Cu") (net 6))
 (segment (start 125.4375 71.4125) (end 125.984 70.866) (width 0.5) (layer "B.Cu") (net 6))
 (segment (start 130.175 68.7705) (end 131.1275 67.818) (width 0.5) (layer "B.Cu") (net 6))
 (segment (start 131.953 61.595) (end 124.333 61.595) (width 0.5) (layer "B.Cu") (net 8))
 (segment (start 123.698 45.72) (end 127 45.72) (width 0.5) (layer "B.Cu") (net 8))
 (segment (start 124.333 61.595) (end 123.305 60.567) (width 0.5) (layer "B.Cu") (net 8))
 (segment (start 123.305 60.567) (end 123.305 46.113) (width 0.5) (layer "B.Cu") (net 8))
 (segment (start 123.305 46.113) (end 123.698 45.72) (width 0.5) (layer "B.Cu") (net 8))
 (segment (start 131.7056 44.184) (end 148.832 44.184) (width 0.5) (layer "B.Cu") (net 5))
 (segment (start 148.832 44.184) (end 150.368 45.72) (width 0.5) (layer "B.Cu") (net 5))
 (segment (start 150.368 45.72) (end 150.368 62.992) (width 0.5) (layer "B.Cu") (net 5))
 (segment (start 150.368 62.992) (end 147.32 66.04) (width 0.5) (layer "B.Cu") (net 5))
 (segment (start 127 48.8896) (end 131.7056 44.184) (width 0.5) (layer "B.Cu") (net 5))
 (segment (start 125.095 59.69) (end 125.095 56.515) (width 0.5) (layer "B.Cu") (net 4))
 (segment (start 125.095 56.515) (end 125.73 55.88) (width 0.5) (layer "B.Cu") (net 4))
 (segment (start 125.73 55.88) (end 127 55.88) (width 0.5) (layer "B.Cu") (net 4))
 (segment (start 133.938 54.356) (end 128.35 59.944) (width 0.5) (layer "B.Cu") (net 4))
 (segment (start 128.35 59.944) (end 125.349 59.944) (width 0.5) (layer "B.Cu") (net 4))
 (segment (start 142.24 55.88) (end 140.716 54.356) (width 0.5) (layer "B.Cu") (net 4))
 (segment (start 125.349 59.944) (end 125.095 59.69) (width 0.5) (layer "B.Cu") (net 4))
 (segment (start 142.24 61.569) (end 142.24 55.88) (width 0.5) (layer "B.Cu") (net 4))
 (segment (start 140.716 54.356) (end 133.938 54.356) (width 0.5) (layer "B.Cu") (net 4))
 (segment (start 133.477 53.467) (end 146.431 53.467) (width 0.5) (layer "B.Cu") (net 3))
 (segment (start 146.431 53.467) (end 147.32 54.356) (width 0.5) (layer "B.Cu") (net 3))
 (segment (start 127 58.42) (end 128.524 58.42) (width 0.5) (layer "B.Cu") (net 3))
 (segment (start 147.32 54.356) (end 147.32 55.88) (width 0.5) (layer "B.Cu") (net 3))
 (segment (start 128.524 58.42) (end 133.477 53.467) (width 0.5) (layer "B.Cu") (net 3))
 (segment (start 145.034 46.101) (end 145.415 45.72) (width 0.5) (layer "B.Cu") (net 2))
 (segment (start 124.968 60.833) (end 124.206 60.071) (width 0.5) (layer "B.Cu") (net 2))
 (segment (start 125.222 68.58) (end 124.968 68.326) (width 0.5) (layer "B.Cu") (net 2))
 (segment (start 133.731 60.198) (end 129.54 60.198) (width 0.5) (layer "B.Cu") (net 2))
 (segment (start 124.587 52.705) (end 144.145 52.705) (width 0.5) (layer "B.Cu") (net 2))
 (segment (start 134.112 60.579) (end 133.731 60.198) (width 0.5) (layer "B.Cu") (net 2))
 (segment (start 127 68.58) (end 125.222 68.58) (width 0.5) (layer "B.Cu") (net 2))
 (segment (start 128.905 60.833) (end 124.968 60.833) (width 0.5) (layer "B.Cu") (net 2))
 (segment (start 125.857 63.119) (end 133.858 63.119) (width 0.5) (layer "B.Cu") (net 2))
 (segment (start 134.112 62.865) (end 134.112 60.579) (width 0.5) (layer "B.Cu") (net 2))
 (segment (start 129.54 60.198) (end 128.905 60.833) (width 0.5) (layer "B.Cu") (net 2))
 (segment (start 124.206 53.086) (end 124.587 52.705) (width 0.5) (layer "B.Cu") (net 2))
 (segment (start 133.858 63.119) (end 134.112 62.865) (width 0.5) (layer "B.Cu") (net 2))
 (segment (start 124.968 64.008) (end 125.857 63.119) (width 0.5) (layer "B.Cu") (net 2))
 (segment (start 145.415 45.72) (end 147.32 45.72) (width 0.5) (layer "B.Cu") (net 2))
 (segment (start 124.968 68.326) (end 124.968 64.008) (width 0.5) (layer "B.Cu") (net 2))
 (segment (start 144.145 52.705) (end 145.034 51.816) (width 0.5) (layer "B.Cu") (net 2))
 (segment (start 124.206 60.071) (end 124.206 53.086) (width 0.5) (layer "B.Cu") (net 2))
 (segment (start 145.034 51.816) (end 145.034 46.101) (width 0.5) (layer "B.Cu") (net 2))
 (segment (start 130.81 66.675) (end 130.175 66.04) (width 0.5) (layer "B.Cu") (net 10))
 (segment (start 132.08 67.03) (end 131.725 66.675) (width 0.5) (layer "B.Cu") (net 10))
 (segment (start 131.725 66.675) (end 130.81 66.675) (width 0.5) (layer "B.Cu") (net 10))
 (segment (start 130.175 66.04) (end 127 66.04) (width 0.5) (layer "B.Cu") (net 10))
 (segment (start 137.16 55.88) (end 135.636 55.88) (width 0.5) (layer "B.Cu") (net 9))
 (segment (start 135.128 60.96) (end 135.737 61.569) (width 0.5) (layer "B.Cu") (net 9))
 (segment (start 135.636 55.88) (end 135.128 56.388) (width 0.5) (layer "B.Cu") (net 9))
 (segment (start 135.128 56.388) (end 135.128 60.96) (width 0.5) (layer "B.Cu") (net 9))
 (segment (start 135.737 61.569) (end 138.557 61.569) (width 0.5) (layer "B.Cu") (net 9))
 (segment (start 139.065 70.485) (end 139.065 72.325) (width 0.5) (layer "B.Cu") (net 17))
 (segment (start 132.422 69.788) (end 138.368 69.788) (width 0.5) (layer "B.Cu") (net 17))
 (segment (start 138.368 69.788) (end 139.065 70.485) (width 0.5) (layer "B.Cu") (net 17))
 (segment (start 132.08 70.13) (end 132.422 69.788) (width 0.5) (layer "B.Cu") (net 17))
 (segment (start 136.525 72.325) (end 136.525 73.299999) (width 0.5) (layer "B.Cu") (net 18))
 (segment (start 142.24 73.152) (end 142.24 64.669) (width 0.5) (layer "B.Cu") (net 18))
 (segment (start 141.478 73.914) (end 142.24 73.152) (width 0.5) (layer "B.Cu") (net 18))
 (segment (start 137.139001 73.914) (end 141.478 73.914) (width 0.5) (layer "B.Cu") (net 18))
 (segment (start 136.525 73.299999) (end 137.139001 73.914) (width 0.5) (layer "B.Cu") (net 18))
 (segment (start 135.89 64.77) (end 132.689 64.77) (width 0.5) (layer "B.Cu") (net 15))
 (segment (start 136.525 65.405) (end 135.89 64.77) (width 0.5) (layer "B.Cu") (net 15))
 (segment (start 136.525 67.375) (end 136.525 65.405) (width 0.5) (layer "B.Cu") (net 15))
 (segment (start 132.689 64.77) (end 132.588 64.669) (width 0.5) (layer "B.Cu") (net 15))
 (segment (start 137.287 68.961) (end 134.62 68.961) (width 0.5) (layer "B.Cu") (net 11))
 (segment (start 134.62 68.961) (end 134.239 68.58) (width 0.5) (layer "B.Cu") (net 11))
 (segment (start 133.096 71.12) (end 133.35 71.374) (width 0.5) (layer "B.Cu") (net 11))
 (segment (start 137.795 67.945) (end 137.795 67.375) (width 0.5) (layer "B.Cu") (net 11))
 (segment (start 130.937 69.156976) (end 130.937 70.358) (width 0.5) (layer "B.Cu") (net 11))
 (segment (start 137.795 68.453) (end 137.287 68.961) (width 0.5) (layer "B.Cu") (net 11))
 (segment (start 131.699 71.12) (end 133.096 71.12) (width 0.5) (layer "B.Cu") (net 11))
 (segment (start 133.35 71.374) (end 133.35 74.0965) (width 0.5) (layer "B.Cu") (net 11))
 (segment (start 137.795 67.375) (end 137.795 68.453) (width 0.5) (layer "B.Cu") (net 11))
 (segment (start 130.937 70.358) (end 131.699 71.12) (width 0.5) (layer "B.Cu") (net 11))
 (segment (start 131.513976 68.58) (end 130.937 69.156976) (width 0.5) (layer "B.Cu") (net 11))
 (segment (start 134.239 68.58) (end 131.513976 68.58) (width 0.5) (layer "B.Cu") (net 11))
 (segment (start 133.35 74.0965) (end 132.395 75.0515) (width 0.5) (layer "B.Cu") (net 11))
 (segment (start 130.495 74.7975) (end 130.495 76.331) (width 0.5) (layer "B.Cu") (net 12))
 (segment (start 130.495 76.331) (end 130.175 76.651) (width 0.5) (layer "B.Cu") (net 12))
 (segment (start 137.795 71.12) (end 137.287 70.612) (width 0.5) (layer "B.Cu") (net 7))
 (segment (start 146.304 91.948) (end 145.796 92.456) (width 0.5) (layer "B.Cu") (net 7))
 (segment (start 137.795 72.325) (end 137.795 71.12) (width 0.5) (layer "B.Cu") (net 7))
 (segment (start 134.493 70.612) (end 134.15 70.955) (width 0.5) (layer "B.Cu") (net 7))
 (segment (start 146.304 76.2) (end 146.304 91.948) (width 0.5) (layer "B.Cu") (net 7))
 (segment (start 126.365 91.948) (end 126.365 81.915) (width 0.5) (layer "B.Cu") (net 7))
 (segment (start 145.796 92.456) (end 126.873 92.456) (width 0.5) (layer "B.Cu") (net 7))
 (segment (start 137.287 70.612) (end 134.493 70.612) (width 0.5) (layer "B.Cu") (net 7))
 (segment (start 134.15 70.955) (end 134.15 74.0975) (width 0.5) (layer "B.Cu") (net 7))
 (segment (start 135.7445 75.692) (end 145.796 75.692) (width 0.5) (layer "B.Cu") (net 7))
 (segment (start 134.15 74.0975) (end 135.7445 75.692) (width 0.5) (layer "B.Cu") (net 7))
 (segment (start 145.796 75.692) (end 146.304 76.2) (width 0.5) (layer "B.Cu") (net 7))
 (segment (start 126.873 92.456) (end 126.365 91.948) (width 0.5) (layer "B.Cu") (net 7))
 (segment (start 139.065 67.375) (end 139.192 67.248) (width 0.5) (layer "B.Cu") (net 16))
 (segment (start 138.557 64.669) (end 138.557 65.024) (width 0.5) (layer "B.Cu") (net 16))
 (segment (start 138.557 65.024) (end 139.065 65.532) (width 0.5) (layer "B.Cu") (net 16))
 (segment (start 139.065 65.532) (end 139.065 67.375) (width 0.5) (layer "B.Cu") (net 16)))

